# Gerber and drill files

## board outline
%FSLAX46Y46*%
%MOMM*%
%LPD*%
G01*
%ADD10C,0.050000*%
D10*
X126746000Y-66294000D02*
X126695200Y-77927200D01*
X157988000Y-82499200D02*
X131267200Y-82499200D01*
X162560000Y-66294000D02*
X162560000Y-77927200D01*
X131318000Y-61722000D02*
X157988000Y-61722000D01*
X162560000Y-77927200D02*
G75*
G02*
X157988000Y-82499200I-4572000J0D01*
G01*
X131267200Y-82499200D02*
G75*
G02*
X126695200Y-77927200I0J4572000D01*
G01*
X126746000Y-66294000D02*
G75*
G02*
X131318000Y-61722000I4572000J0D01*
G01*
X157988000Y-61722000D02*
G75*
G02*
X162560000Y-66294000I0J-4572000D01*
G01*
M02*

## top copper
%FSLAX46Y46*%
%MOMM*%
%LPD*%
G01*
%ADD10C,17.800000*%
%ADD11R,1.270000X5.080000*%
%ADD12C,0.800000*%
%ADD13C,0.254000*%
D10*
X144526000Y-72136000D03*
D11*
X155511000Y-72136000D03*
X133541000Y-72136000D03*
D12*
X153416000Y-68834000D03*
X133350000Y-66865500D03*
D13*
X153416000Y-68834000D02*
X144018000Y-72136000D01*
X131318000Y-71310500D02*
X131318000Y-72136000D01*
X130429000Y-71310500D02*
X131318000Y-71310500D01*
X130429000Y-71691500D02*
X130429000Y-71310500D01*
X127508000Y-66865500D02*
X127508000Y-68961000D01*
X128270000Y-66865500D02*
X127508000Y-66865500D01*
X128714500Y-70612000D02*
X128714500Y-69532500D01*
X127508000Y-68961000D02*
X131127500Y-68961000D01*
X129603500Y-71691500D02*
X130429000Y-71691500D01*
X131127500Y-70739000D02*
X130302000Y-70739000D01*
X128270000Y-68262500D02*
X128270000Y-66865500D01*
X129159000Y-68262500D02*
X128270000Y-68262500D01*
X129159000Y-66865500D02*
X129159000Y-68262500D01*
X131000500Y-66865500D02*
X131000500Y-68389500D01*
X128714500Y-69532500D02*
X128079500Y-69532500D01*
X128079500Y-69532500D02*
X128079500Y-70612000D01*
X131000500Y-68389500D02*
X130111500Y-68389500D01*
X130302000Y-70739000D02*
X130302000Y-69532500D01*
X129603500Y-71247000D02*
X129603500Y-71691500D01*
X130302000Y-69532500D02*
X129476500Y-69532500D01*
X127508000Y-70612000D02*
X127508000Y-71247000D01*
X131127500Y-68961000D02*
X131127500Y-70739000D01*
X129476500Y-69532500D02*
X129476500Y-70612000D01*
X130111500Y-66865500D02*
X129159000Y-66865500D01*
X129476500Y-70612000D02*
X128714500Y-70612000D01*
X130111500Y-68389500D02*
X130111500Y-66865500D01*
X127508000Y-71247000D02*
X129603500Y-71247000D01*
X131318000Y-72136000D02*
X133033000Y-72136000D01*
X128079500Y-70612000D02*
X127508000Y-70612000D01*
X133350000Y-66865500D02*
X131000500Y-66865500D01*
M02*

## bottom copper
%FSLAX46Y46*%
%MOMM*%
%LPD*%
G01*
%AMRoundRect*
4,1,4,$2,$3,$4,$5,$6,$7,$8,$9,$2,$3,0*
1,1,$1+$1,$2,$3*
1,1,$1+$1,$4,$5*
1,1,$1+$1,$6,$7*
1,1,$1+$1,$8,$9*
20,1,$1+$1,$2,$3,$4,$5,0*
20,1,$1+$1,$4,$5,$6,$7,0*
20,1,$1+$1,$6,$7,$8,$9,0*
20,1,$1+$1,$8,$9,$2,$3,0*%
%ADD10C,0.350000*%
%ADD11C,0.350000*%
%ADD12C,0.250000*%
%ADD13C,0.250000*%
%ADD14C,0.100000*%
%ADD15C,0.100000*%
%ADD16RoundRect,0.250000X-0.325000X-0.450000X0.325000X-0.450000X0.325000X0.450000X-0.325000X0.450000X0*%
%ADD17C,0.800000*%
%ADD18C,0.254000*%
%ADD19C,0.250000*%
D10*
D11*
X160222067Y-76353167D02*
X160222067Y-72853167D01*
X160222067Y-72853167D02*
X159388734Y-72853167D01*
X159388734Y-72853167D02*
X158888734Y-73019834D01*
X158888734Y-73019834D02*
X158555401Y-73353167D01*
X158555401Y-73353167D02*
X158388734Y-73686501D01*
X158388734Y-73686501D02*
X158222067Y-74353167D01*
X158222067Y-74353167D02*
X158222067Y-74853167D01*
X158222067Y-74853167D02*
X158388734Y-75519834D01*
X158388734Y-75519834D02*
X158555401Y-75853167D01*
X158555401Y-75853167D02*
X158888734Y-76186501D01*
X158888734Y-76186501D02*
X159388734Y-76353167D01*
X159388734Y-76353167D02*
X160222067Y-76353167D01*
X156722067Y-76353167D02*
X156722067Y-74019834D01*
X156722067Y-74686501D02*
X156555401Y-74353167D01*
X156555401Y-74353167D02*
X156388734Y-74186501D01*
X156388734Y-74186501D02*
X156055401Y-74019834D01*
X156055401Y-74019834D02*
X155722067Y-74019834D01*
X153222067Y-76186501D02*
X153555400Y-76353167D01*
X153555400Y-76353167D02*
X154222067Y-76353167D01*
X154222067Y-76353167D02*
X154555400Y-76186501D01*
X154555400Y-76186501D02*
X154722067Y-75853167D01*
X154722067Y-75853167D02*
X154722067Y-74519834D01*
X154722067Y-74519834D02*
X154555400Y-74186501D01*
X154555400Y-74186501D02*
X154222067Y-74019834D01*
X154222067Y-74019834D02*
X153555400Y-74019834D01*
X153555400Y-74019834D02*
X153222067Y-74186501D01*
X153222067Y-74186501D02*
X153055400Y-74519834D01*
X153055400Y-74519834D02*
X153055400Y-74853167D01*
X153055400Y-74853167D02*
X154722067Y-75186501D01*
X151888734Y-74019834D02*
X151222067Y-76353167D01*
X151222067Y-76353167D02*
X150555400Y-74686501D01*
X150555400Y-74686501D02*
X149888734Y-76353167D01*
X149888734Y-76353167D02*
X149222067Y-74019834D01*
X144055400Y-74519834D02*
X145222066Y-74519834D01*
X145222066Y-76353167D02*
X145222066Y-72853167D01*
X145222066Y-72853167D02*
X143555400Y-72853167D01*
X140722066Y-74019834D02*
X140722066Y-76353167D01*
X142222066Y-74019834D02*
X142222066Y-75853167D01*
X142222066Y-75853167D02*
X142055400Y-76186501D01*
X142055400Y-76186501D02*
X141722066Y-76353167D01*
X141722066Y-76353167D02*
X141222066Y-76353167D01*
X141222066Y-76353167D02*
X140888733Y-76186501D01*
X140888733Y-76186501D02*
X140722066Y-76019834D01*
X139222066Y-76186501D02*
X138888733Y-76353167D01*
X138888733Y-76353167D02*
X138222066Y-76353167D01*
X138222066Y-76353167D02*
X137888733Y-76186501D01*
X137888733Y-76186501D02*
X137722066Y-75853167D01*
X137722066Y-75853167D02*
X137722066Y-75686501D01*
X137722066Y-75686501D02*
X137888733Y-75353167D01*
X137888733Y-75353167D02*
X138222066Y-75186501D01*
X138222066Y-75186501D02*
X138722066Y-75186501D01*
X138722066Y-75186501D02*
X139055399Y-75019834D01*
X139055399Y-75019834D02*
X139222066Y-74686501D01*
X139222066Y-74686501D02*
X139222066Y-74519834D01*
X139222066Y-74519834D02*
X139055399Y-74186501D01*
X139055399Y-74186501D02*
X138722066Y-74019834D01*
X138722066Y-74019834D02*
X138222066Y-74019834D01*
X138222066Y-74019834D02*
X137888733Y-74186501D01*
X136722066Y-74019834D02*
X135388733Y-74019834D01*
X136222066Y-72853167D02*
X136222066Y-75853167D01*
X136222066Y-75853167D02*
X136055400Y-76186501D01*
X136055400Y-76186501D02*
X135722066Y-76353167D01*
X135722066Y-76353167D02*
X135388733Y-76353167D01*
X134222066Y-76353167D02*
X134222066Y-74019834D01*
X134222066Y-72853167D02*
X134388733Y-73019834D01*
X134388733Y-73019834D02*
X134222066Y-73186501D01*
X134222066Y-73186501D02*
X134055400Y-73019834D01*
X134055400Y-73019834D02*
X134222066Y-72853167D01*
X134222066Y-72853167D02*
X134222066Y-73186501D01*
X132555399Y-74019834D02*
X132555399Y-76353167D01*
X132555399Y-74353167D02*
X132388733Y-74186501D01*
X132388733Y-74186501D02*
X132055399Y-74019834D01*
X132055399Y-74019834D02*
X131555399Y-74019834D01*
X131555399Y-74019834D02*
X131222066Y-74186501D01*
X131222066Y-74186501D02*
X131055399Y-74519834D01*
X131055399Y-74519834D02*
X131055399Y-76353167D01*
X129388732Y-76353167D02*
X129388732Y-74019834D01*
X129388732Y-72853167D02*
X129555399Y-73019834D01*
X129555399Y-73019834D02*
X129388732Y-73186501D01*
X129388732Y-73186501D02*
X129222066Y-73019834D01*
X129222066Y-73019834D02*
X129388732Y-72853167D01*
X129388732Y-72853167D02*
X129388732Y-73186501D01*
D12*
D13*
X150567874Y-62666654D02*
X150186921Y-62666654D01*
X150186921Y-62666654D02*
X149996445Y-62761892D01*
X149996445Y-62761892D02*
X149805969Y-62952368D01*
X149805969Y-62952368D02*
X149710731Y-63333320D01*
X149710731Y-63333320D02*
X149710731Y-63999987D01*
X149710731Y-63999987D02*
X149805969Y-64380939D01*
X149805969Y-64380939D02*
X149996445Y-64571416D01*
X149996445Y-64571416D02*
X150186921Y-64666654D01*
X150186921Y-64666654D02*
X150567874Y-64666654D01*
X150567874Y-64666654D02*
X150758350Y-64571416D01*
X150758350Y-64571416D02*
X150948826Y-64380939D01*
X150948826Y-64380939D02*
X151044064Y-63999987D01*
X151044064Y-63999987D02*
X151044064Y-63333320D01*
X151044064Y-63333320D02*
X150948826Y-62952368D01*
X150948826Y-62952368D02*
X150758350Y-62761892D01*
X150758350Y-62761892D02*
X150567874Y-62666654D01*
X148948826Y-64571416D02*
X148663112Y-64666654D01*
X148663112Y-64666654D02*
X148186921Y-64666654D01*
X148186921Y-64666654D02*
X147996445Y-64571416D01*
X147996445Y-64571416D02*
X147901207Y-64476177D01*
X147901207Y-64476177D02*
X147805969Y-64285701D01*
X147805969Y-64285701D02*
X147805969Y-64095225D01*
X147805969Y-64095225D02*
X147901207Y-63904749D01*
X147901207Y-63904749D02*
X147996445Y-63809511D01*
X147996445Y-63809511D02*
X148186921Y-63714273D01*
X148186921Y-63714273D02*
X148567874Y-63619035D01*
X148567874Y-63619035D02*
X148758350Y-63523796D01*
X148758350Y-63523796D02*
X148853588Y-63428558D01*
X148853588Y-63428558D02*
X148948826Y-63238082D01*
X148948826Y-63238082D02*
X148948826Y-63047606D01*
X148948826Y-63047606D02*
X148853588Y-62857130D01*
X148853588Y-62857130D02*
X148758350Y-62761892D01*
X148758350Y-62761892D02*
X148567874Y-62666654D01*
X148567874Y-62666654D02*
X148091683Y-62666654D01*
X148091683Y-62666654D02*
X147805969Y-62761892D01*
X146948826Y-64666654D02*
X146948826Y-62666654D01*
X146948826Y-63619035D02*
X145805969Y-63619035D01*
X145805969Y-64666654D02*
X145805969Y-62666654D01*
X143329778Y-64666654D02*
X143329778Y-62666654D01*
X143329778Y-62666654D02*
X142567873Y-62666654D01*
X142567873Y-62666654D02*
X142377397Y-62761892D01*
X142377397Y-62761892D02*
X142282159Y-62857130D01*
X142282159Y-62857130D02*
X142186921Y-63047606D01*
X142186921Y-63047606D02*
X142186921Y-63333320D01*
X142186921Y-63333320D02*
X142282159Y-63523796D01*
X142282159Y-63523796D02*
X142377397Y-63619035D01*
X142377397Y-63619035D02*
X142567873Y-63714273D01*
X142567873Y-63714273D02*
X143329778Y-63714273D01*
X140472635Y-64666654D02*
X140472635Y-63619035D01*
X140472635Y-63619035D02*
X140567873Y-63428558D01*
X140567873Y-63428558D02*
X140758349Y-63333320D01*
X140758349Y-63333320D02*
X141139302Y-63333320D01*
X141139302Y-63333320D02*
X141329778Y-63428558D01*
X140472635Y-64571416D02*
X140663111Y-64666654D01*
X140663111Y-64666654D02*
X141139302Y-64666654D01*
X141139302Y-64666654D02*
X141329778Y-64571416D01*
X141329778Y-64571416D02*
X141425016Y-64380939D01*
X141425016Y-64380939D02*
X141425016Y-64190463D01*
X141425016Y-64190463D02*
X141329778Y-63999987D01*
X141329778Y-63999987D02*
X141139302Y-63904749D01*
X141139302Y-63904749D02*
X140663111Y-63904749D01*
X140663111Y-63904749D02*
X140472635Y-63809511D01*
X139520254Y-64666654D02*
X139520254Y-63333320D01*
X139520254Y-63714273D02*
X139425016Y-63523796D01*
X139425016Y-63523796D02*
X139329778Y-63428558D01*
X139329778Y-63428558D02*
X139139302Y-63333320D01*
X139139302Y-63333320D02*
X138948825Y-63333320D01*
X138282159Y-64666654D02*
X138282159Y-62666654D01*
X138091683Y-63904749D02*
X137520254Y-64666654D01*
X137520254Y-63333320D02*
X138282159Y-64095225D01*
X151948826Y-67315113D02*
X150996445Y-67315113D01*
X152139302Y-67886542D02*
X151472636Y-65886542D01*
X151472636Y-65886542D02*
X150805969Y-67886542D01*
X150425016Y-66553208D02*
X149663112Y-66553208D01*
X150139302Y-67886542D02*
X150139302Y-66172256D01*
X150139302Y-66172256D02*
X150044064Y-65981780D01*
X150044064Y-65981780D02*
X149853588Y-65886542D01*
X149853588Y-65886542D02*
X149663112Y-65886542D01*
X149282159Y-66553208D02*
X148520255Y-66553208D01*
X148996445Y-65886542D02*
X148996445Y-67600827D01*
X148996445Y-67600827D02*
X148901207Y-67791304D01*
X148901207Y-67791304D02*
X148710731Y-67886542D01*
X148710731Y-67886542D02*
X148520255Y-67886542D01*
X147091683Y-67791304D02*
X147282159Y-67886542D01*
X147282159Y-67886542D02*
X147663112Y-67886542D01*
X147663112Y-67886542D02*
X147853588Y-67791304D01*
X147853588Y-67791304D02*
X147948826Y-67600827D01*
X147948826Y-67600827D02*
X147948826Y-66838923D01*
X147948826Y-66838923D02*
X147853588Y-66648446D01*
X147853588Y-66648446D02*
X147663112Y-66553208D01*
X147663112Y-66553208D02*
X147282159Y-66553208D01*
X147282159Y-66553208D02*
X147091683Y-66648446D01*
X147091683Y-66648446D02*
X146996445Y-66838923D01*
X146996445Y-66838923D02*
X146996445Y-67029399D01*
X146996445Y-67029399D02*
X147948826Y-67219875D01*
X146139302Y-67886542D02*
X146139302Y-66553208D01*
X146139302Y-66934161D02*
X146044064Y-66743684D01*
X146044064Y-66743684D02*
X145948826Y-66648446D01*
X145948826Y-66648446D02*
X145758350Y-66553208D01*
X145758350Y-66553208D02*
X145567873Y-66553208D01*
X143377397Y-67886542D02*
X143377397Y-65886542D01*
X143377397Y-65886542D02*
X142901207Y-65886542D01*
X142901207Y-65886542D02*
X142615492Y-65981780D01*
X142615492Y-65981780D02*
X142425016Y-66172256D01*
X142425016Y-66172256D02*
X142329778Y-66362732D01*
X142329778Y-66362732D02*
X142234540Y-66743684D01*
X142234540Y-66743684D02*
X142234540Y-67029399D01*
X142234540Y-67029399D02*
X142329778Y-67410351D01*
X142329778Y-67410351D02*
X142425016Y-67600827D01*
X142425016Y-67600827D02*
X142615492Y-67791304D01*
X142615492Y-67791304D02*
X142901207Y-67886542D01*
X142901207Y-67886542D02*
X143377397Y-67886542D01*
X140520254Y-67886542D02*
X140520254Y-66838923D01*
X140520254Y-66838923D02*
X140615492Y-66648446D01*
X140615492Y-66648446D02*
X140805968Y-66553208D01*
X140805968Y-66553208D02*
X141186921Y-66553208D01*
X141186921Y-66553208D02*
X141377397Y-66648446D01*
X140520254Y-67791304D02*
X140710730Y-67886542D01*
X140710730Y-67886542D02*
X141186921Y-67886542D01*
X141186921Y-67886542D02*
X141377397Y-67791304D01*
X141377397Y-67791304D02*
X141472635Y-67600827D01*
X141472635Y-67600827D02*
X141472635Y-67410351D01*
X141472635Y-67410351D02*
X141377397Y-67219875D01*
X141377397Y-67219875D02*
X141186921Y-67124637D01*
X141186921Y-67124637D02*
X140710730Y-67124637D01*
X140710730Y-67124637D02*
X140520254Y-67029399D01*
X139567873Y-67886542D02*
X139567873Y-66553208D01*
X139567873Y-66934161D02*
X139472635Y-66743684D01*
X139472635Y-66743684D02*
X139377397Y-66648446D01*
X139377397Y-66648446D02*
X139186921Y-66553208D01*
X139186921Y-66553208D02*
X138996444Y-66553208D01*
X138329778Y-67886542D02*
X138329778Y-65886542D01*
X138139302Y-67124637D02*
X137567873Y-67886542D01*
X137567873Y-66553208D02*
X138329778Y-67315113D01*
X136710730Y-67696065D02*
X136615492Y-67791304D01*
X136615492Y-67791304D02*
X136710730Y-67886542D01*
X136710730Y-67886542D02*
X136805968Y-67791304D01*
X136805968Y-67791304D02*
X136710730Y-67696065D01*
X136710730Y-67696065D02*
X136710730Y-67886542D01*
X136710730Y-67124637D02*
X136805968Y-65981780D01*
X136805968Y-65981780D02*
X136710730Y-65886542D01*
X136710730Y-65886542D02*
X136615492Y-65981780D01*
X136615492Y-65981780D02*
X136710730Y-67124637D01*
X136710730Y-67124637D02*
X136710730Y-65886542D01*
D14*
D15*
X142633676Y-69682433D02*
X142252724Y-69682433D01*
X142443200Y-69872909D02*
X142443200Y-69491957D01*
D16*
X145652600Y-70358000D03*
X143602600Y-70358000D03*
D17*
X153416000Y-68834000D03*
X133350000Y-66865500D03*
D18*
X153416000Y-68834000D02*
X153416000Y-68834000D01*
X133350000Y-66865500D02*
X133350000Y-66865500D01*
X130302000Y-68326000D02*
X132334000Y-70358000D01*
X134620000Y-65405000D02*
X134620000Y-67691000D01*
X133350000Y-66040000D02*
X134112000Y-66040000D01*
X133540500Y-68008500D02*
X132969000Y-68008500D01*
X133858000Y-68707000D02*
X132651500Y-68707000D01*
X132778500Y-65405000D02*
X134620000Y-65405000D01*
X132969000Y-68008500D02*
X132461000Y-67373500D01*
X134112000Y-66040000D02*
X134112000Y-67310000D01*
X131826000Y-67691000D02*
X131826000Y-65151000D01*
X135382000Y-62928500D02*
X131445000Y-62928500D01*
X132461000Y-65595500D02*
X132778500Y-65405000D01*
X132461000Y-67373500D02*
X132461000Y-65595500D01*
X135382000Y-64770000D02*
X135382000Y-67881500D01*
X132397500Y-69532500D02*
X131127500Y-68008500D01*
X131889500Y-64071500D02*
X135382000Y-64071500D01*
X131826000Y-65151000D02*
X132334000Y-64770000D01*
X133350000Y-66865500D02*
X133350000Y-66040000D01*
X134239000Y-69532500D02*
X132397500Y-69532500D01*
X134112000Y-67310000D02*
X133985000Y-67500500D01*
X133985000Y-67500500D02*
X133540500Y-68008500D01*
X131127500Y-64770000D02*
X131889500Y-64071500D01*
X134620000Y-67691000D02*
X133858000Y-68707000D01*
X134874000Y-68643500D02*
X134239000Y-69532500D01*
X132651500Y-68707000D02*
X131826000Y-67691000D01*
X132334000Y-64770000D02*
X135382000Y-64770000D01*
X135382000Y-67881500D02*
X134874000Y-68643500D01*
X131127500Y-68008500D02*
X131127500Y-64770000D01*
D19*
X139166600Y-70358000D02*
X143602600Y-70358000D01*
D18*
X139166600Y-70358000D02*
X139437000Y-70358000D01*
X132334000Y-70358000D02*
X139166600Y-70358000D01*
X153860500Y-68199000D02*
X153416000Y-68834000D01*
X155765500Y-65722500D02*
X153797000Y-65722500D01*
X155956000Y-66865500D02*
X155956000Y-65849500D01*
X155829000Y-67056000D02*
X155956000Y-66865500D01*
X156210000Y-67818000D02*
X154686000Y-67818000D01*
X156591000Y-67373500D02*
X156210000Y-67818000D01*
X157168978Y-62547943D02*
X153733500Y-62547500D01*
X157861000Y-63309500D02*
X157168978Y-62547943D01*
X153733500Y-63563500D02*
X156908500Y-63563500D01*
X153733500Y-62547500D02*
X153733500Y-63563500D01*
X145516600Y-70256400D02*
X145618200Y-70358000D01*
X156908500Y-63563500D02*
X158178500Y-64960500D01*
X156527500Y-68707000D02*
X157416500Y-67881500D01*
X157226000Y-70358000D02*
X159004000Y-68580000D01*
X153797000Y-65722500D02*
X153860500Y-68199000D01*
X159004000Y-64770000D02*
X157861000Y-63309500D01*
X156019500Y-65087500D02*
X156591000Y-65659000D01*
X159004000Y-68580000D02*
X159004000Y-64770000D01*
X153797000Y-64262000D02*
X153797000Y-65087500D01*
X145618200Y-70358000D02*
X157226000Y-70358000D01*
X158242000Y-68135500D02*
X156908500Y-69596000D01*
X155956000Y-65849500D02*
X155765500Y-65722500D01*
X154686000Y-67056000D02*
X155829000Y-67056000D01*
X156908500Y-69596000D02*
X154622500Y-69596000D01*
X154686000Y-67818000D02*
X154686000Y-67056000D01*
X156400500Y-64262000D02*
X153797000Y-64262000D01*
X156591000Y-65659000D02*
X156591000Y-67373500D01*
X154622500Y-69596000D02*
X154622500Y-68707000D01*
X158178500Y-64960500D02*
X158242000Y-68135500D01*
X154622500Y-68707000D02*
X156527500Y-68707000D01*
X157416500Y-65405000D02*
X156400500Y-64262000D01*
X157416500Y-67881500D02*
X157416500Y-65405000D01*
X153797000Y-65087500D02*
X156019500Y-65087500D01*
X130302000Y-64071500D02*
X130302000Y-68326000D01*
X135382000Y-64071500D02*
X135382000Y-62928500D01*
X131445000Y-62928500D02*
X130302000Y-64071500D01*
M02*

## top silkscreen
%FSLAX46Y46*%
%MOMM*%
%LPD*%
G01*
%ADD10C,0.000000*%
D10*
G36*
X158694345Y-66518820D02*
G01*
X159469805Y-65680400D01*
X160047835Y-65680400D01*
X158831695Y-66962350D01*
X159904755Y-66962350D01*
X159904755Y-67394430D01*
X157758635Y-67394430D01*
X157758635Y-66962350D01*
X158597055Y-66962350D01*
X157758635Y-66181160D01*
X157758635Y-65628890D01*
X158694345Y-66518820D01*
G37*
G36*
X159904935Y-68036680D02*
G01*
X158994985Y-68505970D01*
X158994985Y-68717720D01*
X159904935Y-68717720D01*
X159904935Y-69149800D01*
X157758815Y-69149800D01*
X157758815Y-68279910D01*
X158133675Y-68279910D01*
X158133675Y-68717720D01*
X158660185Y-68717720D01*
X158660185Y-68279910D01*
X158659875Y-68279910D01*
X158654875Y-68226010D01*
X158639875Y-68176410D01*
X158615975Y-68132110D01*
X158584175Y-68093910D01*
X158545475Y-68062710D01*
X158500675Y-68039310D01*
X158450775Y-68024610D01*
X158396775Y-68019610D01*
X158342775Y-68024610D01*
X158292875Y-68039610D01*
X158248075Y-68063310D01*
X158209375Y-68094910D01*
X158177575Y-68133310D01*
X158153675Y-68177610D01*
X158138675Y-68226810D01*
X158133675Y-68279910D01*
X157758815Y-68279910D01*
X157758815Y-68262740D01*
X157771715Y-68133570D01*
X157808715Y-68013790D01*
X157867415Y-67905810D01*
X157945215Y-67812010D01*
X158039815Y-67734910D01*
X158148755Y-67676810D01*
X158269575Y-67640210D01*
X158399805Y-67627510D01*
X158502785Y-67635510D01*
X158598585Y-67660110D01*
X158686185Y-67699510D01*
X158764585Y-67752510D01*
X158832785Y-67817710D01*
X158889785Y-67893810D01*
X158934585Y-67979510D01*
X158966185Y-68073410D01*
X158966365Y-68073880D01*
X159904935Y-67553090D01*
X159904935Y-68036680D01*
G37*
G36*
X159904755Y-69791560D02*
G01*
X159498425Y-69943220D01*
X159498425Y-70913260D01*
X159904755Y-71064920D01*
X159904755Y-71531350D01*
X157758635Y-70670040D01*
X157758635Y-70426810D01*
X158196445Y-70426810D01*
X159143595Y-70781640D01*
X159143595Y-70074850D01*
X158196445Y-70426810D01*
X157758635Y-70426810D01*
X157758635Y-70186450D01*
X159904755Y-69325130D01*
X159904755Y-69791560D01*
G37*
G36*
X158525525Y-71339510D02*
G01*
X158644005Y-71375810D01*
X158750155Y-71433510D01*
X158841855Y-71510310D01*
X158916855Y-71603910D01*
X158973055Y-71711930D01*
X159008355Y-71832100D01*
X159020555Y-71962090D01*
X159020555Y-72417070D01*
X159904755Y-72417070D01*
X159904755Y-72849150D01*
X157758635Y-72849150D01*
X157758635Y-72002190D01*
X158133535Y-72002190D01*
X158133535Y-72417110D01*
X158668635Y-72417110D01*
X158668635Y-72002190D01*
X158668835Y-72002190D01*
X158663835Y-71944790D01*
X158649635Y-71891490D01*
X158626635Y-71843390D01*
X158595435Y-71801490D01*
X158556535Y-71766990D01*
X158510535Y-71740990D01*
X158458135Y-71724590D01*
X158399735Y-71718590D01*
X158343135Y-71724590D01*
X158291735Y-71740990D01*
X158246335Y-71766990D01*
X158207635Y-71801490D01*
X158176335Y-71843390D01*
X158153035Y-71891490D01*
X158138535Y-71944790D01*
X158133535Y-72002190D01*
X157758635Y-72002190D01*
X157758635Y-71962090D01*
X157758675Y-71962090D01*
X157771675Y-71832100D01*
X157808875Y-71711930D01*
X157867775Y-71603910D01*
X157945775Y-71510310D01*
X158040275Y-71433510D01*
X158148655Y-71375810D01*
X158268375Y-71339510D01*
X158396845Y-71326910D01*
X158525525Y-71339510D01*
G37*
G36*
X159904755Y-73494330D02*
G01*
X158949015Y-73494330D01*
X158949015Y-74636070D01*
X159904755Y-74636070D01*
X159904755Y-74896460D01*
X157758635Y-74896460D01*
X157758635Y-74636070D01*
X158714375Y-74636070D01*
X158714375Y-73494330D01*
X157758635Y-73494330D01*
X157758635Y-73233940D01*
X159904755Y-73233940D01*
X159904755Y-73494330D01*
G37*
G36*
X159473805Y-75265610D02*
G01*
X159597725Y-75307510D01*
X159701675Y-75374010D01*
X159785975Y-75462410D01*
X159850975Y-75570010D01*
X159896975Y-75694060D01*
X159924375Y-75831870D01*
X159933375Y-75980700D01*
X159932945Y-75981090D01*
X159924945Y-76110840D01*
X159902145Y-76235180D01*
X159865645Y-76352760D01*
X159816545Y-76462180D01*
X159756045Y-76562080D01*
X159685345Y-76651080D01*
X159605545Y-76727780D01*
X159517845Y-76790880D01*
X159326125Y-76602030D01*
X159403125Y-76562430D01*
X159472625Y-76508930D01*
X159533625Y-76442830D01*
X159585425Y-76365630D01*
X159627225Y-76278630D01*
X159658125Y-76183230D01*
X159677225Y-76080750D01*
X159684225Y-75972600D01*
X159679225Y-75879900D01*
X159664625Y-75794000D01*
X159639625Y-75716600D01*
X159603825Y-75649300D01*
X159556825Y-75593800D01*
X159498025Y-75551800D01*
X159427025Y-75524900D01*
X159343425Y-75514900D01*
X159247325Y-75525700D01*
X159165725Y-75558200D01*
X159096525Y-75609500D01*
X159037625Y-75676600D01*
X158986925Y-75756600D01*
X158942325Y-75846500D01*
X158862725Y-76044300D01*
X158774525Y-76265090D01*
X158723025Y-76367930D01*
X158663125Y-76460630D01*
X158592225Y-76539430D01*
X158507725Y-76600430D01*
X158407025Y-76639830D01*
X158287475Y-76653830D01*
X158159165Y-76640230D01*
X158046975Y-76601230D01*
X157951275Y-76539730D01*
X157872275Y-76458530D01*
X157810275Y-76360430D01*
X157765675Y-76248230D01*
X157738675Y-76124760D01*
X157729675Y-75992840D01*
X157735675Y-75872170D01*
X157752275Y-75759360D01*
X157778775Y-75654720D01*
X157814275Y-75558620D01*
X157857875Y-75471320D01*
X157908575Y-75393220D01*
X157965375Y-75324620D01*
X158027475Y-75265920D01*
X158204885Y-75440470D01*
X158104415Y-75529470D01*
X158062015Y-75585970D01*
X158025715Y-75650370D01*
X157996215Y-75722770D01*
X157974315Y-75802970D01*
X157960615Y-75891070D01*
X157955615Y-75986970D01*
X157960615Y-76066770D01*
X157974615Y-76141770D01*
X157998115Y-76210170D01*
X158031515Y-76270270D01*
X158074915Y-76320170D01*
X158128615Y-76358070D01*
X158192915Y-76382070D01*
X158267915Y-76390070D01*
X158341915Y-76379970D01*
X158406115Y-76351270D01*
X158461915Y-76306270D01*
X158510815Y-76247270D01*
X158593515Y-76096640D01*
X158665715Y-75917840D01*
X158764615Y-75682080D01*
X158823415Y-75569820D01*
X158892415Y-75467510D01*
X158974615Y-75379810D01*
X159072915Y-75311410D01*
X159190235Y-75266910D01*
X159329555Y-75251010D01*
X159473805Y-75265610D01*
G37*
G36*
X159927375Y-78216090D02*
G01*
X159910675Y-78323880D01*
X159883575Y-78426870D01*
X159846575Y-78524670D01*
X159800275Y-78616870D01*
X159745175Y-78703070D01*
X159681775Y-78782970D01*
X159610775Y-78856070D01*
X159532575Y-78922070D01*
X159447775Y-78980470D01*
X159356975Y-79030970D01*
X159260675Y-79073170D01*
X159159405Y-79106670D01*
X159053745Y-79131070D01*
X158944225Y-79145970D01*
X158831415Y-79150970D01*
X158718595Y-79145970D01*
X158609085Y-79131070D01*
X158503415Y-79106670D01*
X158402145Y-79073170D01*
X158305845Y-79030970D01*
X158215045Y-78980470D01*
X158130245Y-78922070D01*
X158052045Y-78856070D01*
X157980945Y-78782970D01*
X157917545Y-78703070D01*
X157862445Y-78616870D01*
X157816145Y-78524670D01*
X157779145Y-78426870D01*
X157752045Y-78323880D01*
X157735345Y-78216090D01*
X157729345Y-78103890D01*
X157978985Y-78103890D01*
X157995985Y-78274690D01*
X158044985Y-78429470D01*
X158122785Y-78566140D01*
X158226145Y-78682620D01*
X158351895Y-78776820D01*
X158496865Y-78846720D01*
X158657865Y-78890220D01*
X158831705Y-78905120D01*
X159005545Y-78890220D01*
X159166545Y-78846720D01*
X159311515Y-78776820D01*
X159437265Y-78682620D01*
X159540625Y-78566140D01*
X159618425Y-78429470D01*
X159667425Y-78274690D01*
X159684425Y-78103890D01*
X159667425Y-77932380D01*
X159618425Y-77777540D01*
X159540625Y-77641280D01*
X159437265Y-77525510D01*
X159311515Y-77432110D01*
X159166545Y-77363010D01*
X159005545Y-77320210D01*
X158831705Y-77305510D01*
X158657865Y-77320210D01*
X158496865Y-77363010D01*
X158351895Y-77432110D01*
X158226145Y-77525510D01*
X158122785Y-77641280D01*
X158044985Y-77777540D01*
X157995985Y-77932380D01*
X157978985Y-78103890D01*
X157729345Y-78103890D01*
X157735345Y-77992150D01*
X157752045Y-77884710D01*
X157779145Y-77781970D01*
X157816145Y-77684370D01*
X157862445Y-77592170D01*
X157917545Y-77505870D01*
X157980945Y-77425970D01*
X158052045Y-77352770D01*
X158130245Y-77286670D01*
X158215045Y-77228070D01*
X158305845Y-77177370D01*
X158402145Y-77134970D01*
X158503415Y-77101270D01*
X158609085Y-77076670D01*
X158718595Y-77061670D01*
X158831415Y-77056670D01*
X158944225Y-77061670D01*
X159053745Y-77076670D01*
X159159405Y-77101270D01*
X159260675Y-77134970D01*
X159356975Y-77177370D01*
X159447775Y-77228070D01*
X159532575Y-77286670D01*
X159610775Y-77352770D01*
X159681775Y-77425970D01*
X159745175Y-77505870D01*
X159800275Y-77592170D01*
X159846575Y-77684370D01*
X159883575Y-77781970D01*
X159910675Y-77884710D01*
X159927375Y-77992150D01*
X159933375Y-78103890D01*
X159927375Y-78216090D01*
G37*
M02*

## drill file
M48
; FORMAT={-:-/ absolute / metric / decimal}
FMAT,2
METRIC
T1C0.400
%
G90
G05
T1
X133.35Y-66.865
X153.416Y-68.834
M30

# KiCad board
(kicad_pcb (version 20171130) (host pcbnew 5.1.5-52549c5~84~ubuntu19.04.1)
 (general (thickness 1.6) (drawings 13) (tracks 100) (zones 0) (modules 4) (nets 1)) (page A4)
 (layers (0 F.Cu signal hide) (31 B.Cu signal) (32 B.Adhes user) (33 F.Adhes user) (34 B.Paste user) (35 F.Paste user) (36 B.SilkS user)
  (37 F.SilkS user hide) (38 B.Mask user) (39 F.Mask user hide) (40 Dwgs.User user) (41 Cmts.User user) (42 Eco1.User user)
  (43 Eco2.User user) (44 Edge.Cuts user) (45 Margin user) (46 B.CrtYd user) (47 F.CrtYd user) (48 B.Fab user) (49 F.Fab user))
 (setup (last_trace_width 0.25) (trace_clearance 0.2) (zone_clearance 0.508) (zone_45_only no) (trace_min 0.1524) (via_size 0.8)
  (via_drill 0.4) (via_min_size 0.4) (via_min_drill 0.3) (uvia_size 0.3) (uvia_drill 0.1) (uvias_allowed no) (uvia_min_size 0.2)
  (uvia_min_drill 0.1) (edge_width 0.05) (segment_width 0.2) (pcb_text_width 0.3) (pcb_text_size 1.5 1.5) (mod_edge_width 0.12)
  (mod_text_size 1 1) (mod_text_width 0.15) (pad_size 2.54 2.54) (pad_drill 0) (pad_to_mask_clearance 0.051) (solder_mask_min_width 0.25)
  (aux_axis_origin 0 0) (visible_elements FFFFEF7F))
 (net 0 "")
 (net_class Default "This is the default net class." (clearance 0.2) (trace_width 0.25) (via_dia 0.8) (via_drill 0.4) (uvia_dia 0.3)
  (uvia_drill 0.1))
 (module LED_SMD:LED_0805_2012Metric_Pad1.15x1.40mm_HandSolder (layer B.Cu) (at 144.6276 70.358)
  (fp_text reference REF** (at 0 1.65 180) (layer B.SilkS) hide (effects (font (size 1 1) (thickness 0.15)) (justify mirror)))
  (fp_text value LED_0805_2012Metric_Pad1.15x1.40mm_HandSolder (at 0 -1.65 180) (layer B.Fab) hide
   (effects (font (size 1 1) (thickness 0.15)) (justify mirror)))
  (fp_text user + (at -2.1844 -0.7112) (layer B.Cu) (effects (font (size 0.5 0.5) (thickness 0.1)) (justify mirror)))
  (pad 2 smd roundrect (at 1.025 0) (size 1.15 1.4) (layers B.Cu B.Paste B.Mask) (roundrect_rratio 0.217391))
  (pad 1 smd roundrect (at -1.025 0) (size 1.15 1.4) (layers B.Cu B.Paste B.Mask) (roundrect_rratio 0.217391)))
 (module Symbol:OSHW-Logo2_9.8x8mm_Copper (layer F.Cu) (at 131.572 79.502)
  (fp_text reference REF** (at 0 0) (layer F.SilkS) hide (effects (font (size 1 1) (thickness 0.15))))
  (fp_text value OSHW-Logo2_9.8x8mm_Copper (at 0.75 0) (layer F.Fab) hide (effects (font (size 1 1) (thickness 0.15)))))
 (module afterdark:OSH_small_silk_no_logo (layer F.Cu) (at 151.638 72.39 90)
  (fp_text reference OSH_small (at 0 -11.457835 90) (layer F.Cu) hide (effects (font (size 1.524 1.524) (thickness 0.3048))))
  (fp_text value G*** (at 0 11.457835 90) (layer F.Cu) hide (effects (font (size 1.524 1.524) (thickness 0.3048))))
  (fp_poly
   (pts (xy 6.76111 6.120635) (xy 6.20884 6.120635) (xy 5.42765 6.959055) (xy 5.42765 6.120635) (xy 4.99557 6.120635) (xy 4.99557 8.266755)
    (xy 5.42765 8.266755) (xy 5.42765 7.193695) (xy 6.7096 8.409835) (xy 6.7096 7.831805) (xy 5.87118 7.056345) (xy 6.76111 6.120635))
   (layer F.SilkS) (width 0))
  (fp_poly
   (pts (xy 4.31659 7.328185) (xy 4.11009 7.022185) (xy 3.67228 7.022185) (xy 3.67228 6.495675) (xy 4.11009 6.495675) (xy 4.16319 6.500675)
    (xy 4.21239 6.515675) (xy 4.25669 6.539575) (xy 4.29509 6.571375) (xy 4.32669 6.610075) (xy 4.35039 6.654875) (xy 4.36539 6.704775)
    (xy 4.37039 6.758775) (xy 4.36539 6.812775) (xy 4.35069 6.862675) (xy 4.32729 6.907475) (xy 4.29609 6.946175) (xy 4.25789 6.977975)
    (xy 4.21359 7.001875) (xy 4.16399 7.016875) (xy 4.11009 7.021875) (xy 4.11009 7.022185) (xy 4.31659 7.328185) (xy 4.41049 7.296585)
    (xy 4.49619 7.251785) (xy 4.57229 7.194785) (xy 4.63749 7.126585) (xy 4.69049 7.048185) (xy 4.72989 6.960585) (xy 4.75449 6.864785)
    (xy 4.76249 6.761805) (xy 4.74979 6.631575) (xy 4.71319 6.510755) (xy 4.65509 6.401815) (xy 4.57799 6.307215) (xy 4.48419 6.229415)
    (xy 4.37621 6.170715) (xy 4.25643 6.133715) (xy 4.12726 6.120815) (xy 3.2402 6.120815) (xy 3.2402 8.266935) (xy 3.67228 8.266935)
    (xy 3.67228 7.356985) (xy 3.88403 7.356985) (xy 4.35332 8.266935) (xy 4.83691 8.266935) (xy 4.31612 7.328365) (xy 4.31659 7.328185))
   (layer F.SilkS) (width 0))
  (fp_poly
   (pts (xy 2.59844 8.266755) (xy 1.96319 6.558445) (xy 2.31515 7.505595) (xy 1.60836 7.505595) (xy 1.96319 6.558445) (xy 2.59844 8.266755)
    (xy 3.06487 8.266755) (xy 2.20355 6.120635) (xy 1.71996 6.120635) (xy 0.85865 8.266755) (xy 1.32508 8.266755) (xy 1.47674 7.860425)
    (xy 2.44678 7.860425) (xy 2.59844 8.266755))
   (layer F.SilkS) (width 0))
  (fp_poly
   (pts (xy 0.42791 6.120635) (xy -0.02711 6.495535) (xy 0.38781 6.495535) (xy 0.44521 6.500535) (xy 0.49851 6.515035) (xy 0.54661 6.538335)
    (xy 0.58851 6.569635) (xy 0.62301 6.608335) (xy 0.64901 6.653735) (xy 0.66541 6.705135) (xy 0.67141 6.761735) (xy 0.66541 6.820135)
    (xy 0.64901 6.872535) (xy 0.62301 6.918535) (xy 0.58851 6.957435) (xy 0.54661 6.988635) (xy 0.49851 7.011635) (xy 0.44521 7.025835)
    (xy 0.38781 7.030835) (xy 0.38781 7.030635) (xy -0.02711 7.030635) (xy -0.02711 6.495535) (xy 0.42791 6.120635) (xy -0.45915 6.120635)
    (xy -0.45915 8.266755) (xy -0.02707 8.266755) (xy -0.02707 7.382555) (xy 0.42791 7.382555) (xy 0.5579 7.370355) (xy 0.67807 7.335055)
    (xy 0.78609 7.278855) (xy 0.87969 7.203855) (xy 0.95649 7.112155) (xy 1.01419 7.006005) (xy 1.05049 6.887525) (xy 1.06309 6.758845)
    (xy 1.05049 6.630375) (xy 1.01419 6.510655) (xy 0.95649 6.402275) (xy 0.87969 6.307775) (xy 0.78609 6.229775) (xy 0.67807 6.170875)
    (xy 0.5579 6.133675) (xy 0.42791 6.120675) (xy 0.42791 6.120635))
   (layer F.SilkS) (width 0))
  (fp_poly
   (pts (xy -1.10433 6.120635) (xy -1.10433 7.076375) (xy -2.24607 7.076375) (xy -2.24607 6.120635) (xy -2.50646 6.120635)
    (xy -2.50646 8.266755) (xy -2.24607 8.266755) (xy -2.24607 7.311015) (xy -1.10433 7.311015) (xy -1.10433 8.266755)
    (xy -0.84394 8.266755) (xy -0.84394 6.120635) (xy -1.10433 6.120635))
   (layer F.SilkS) (width 0))
  (fp_poly
   (pts (xy -3.5907 8.295375) (xy -3.44187 8.286375) (xy -3.30406 8.258975) (xy -3.18001 8.212975) (xy -3.07241 8.147975)
    (xy -2.98401 8.063675) (xy -2.91751 7.959725) (xy -2.87561 7.835805) (xy -2.86101 7.691555) (xy -2.87691 7.552235)
    (xy -2.92141 7.434915) (xy -2.98981 7.336615) (xy -3.07751 7.254415) (xy -3.17982 7.185415) (xy -3.29208 7.126615)
    (xy -3.52784 7.027715) (xy -3.70664 6.955515) (xy -3.85727 6.872815) (xy -3.91627 6.823915) (xy -3.96127 6.768115)
    (xy -3.98997 6.703915) (xy -4.00007 6.629915) (xy -3.99207 6.554915) (xy -3.96807 6.490615) (xy -3.93017 6.436915)
    (xy -3.88027 6.393515) (xy -3.82017 6.360115) (xy -3.75177 6.336615) (xy -3.67677 6.322615) (xy -3.59697 6.317615)
    (xy -3.50107 6.322615) (xy -3.41297 6.336315) (xy -3.33277 6.358215) (xy -3.26037 6.387715) (xy -3.19597 6.424015)
    (xy -3.13947 6.466415) (xy -3.05047 6.566885) (xy -2.87592 6.389475) (xy -2.93462 6.327375) (xy -3.00322 6.270575)
    (xy -3.08132 6.219875) (xy -3.16862 6.176275) (xy -3.26472 6.140775) (xy -3.36936 6.114275) (xy -3.48217 6.097675)
    (xy -3.60284 6.091675) (xy -3.73476 6.100675) (xy -3.85823 6.127675) (xy -3.97043 6.172275) (xy -4.06853 6.234275)
    (xy -4.14973 6.313275) (xy -4.21123 6.408975) (xy -4.25023 6.521165) (xy -4.26383 6.649475) (xy -4.24983 6.769025)
    (xy -4.21043 6.869725) (xy -4.14943 6.954225) (xy -4.07063 7.025125) (xy -3.97793 7.085025) (xy -3.87509 7.136525) (xy -3.6543 7.224725)
    (xy -3.4565 7.304325) (xy -3.3666 7.348925) (xy -3.2866 7.399625) (xy -3.2195 7.458525) (xy -3.1682 7.527725) (xy -3.1357 7.609325)
    (xy -3.1249 7.705425) (xy -3.1349 7.789025) (xy -3.1618 7.860025) (xy -3.2038 7.918825) (xy -3.2593 7.965825) (xy -3.3266 8.001625)
    (xy -3.404 8.026625) (xy -3.4899 8.041225) (xy -3.5826 8.046225) (xy -3.69075 8.039225) (xy -3.79323 8.020125) (xy -3.88863 7.989225)
    (xy -3.97563 7.947425) (xy -4.05283 7.895625) (xy -4.11893 7.834625) (xy -4.17243 7.765125) (xy -4.21203 7.688125)
    (xy -4.40088 7.879845) (xy -4.33778 7.967545) (xy -4.26108 8.047345) (xy -4.17208 8.118045) (xy -4.07218 8.178545)
    (xy -3.96276 8.227645) (xy -3.84518 8.264145) (xy -3.72084 8.286945) (xy -3.59109 8.294945) (xy -3.5907 8.295375))
   (layer F.SilkS) (width 0))
  (fp_poly
   (pts (xy -5.71389 8.295375) (xy -5.71389 8.046425) (xy -5.88469 8.029425) (xy -6.03947 7.980425) (xy -6.17614 7.902625)
    (xy -6.29262 7.799265) (xy -6.38682 7.673515) (xy -6.45672 7.528545) (xy -6.50022 7.367545) (xy -6.51512 7.193705)
    (xy -6.50022 7.019865) (xy -6.45672 6.858865) (xy -6.38682 6.713895) (xy -6.29262 6.588145) (xy -6.17614 6.484785)
    (xy -6.03947 6.406985) (xy -5.88469 6.357985) (xy -5.71389 6.340985) (xy -5.54238 6.357985) (xy -5.38754 6.406985)
    (xy -5.25128 6.484785) (xy -5.13551 6.588145) (xy -5.04211 6.713895) (xy -4.97301 6.858865) (xy -4.93021 7.019865)
    (xy -4.91551 7.193705) (xy -4.93021 7.367545) (xy -4.97301 7.528545) (xy -5.04211 7.673515) (xy -5.13551 7.799265)
    (xy -5.25128 7.902625) (xy -5.38754 7.980425) (xy -5.54238 8.029425) (xy -5.71389 8.046425) (xy -5.71389 8.295375)
    (xy -5.60215 8.289375) (xy -5.49471 8.272675) (xy -5.39197 8.245575) (xy -5.29437 8.208575) (xy -5.20217 8.162275)
    (xy -5.11587 8.107175) (xy -5.03597 8.043775) (xy -4.96277 7.972775) (xy -4.89667 7.894575) (xy -4.83807 7.809775)
    (xy -4.78737 7.718975) (xy -4.74497 7.622675) (xy -4.71127 7.521405) (xy -4.68667 7.415745) (xy -4.67167 7.306225)
    (xy -4.66667 7.193415) (xy -4.67167 7.080595) (xy -4.68667 6.971085) (xy -4.71127 6.865415) (xy -4.74497 6.764145)
    (xy -4.78737 6.667845) (xy -4.83807 6.577045) (xy -4.89667 6.492245) (xy -4.96277 6.414045) (xy -5.03597 6.342945)
    (xy -5.11587 6.279545) (xy -5.20217 6.224445) (xy -5.29437 6.178145) (xy -5.39197 6.141145) (xy -5.49471 6.114045)
    (xy -5.60215 6.097345) (xy -5.71389 6.091345) (xy -5.82609 6.097345) (xy -5.93388 6.114045) (xy -6.03687 6.141145)
    (xy -6.13467 6.178145) (xy -6.22687 6.224445) (xy -6.31307 6.279545) (xy -6.39297 6.342945) (xy -6.46607 6.414045)
    (xy -6.53207 6.492245) (xy -6.59047 6.577045) (xy -6.64097 6.667845) (xy -6.68317 6.764145) (xy -6.71667 6.865415)
    (xy -6.74107 6.971085) (xy -6.75597 7.080595) (xy -6.76097 7.193415) (xy -6.75597 7.306225) (xy -6.74107 7.415745)
    (xy -6.71667 7.521405) (xy -6.68317 7.622675) (xy -6.64097 7.718975) (xy -6.59047 7.809775) (xy -6.53207 7.894575)
    (xy -6.46607 7.972775) (xy -6.39297 8.043775) (xy -6.31307 8.107175) (xy -6.22687 8.162275) (xy -6.13467 8.208575)
    (xy -6.03687 8.245575) (xy -5.93388 8.272675) (xy -5.82609 8.289375) (xy -5.71389 8.295375))
   (layer F.SilkS) (width 0)))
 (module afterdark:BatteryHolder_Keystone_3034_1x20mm (layer F.Cu) (at 144.526 72.136)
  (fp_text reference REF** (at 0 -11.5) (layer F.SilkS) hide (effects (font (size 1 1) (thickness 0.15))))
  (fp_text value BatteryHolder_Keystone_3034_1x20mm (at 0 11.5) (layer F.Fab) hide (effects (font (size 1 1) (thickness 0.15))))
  (pad 2 smd circle (at 0 0) (size 17.8 17.8) (layers F.Cu F.Mask))
  (pad 1 smd rect (at 10.985 0) (size 1.27 5.08) (layers F.Cu F.Paste F.Mask))
  (pad 1 smd rect (at -10.985 0) (size 1.27 5.08) (layers F.Cu F.Paste F.Mask)))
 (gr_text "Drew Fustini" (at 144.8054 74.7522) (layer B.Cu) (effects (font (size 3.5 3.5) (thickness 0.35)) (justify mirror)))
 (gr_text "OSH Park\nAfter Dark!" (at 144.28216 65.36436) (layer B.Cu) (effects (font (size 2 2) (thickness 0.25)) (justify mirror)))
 (gr_line (start 126.746 66.294) (end 126.6952 77.9272) (layer Edge.Cuts) (width 0.05))
 (gr_line (start 157.988 82.4992) (end 131.2672 82.4992) (layer Edge.Cuts) (width 0.05))
 (gr_line (start 162.56 66.294) (end 162.56 77.9272) (layer Edge.Cuts) (width 0.05))
 (gr_line (start 131.318 61.722) (end 157.988 61.722) (layer Edge.Cuts) (width 0.05))
 (gr_arc (start 157.988 77.9272) (end 157.988 82.4992) (angle -90) (layer Edge.Cuts) (width 0.05))
 (gr_arc (start 131.2672 77.9272) (end 126.6952 77.9272) (angle -90) (layer Edge.Cuts) (width 0.05))
 (gr_arc (start 131.318 66.294) (end 131.318 61.722) (angle -90) (layer Edge.Cuts) (width 0.05))
 (gr_arc (start 157.988 66.294) (end 162.56 66.294) (angle -90) (layer Edge.Cuts) (width 0.05))
 (segment (start 153.416 68.834) (end 153.416 68.834) (width 0.254) (layer B.Cu) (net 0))
 (via (at 153.416 68.834) (size 0.8) (drill 0.4) (layers F.Cu B.Cu) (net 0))
 (segment (start 153.416 68.834) (end 144.018 72.136) (width 0.254) (layer F.Cu) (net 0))
 (segment (start 131.318 71.3105) (end 131.318 72.136) (width 0.254) (layer F.Cu) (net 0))
 (segment (start 130.429 71.3105) (end 131.318 71.3105) (width 0.254) (layer F.Cu) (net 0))
 (segment (start 130.429 71.6915) (end 130.429 71.3105) (width 0.254) (layer F.Cu) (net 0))
 (segment (start 127.508 66.8655) (end 127.508 68.961) (width 0.254) (layer F.Cu) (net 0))
 (segment (start 128.27 66.8655) (end 127.508 66.8655) (width 0.254) (layer F.Cu) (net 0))
 (segment (start 128.7145 70.612) (end 128.7145 69.5325) (width 0.254) (layer F.Cu) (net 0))
 (segment (start 127.508 68.961) (end 131.1275 68.961) (width 0.254) (layer F.Cu) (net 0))
 (segment (start 129.6035 71.6915) (end 130.429 71.6915) (width 0.254) (layer F.Cu) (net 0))
 (segment (start 131.1275 70.739) (end 130.302 70.739) (width 0.254) (layer F.Cu) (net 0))
 (segment (start 128.27 68.2625) (end 128.27 66.8655) (width 0.254) (layer F.Cu) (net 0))
 (segment (start 129.159 68.2625) (end 128.27 68.2625) (width 0.254) (layer F.Cu) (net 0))
 (segment (start 129.159 66.8655) (end 129.159 68.2625) (width 0.254) (layer F.Cu) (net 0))
 (segment (start 131.0005 66.8655) (end 131.0005 68.3895) (width 0.254) (layer F.Cu) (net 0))
 (segment (start 128.7145 69.5325) (end 128.0795 69.5325) (width 0.254) (layer F.Cu) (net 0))
 (segment (start 128.0795 69.5325) (end 128.0795 70.612) (width 0.254) (layer F.Cu) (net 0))
 (segment (start 131.0005 68.3895) (end 130.1115 68.3895) (width 0.254) (layer F.Cu) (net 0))
 (segment (start 130.302 70.739) (end 130.302 69.5325) (width 0.254) (layer F.Cu) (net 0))
 (segment (start 129.6035 71.247) (end 129.6035 71.6915) (width 0.254) (layer F.Cu) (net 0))
 (segment (start 130.302 69.5325) (end 129.4765 69.5325) (width 0.254) (layer F.Cu) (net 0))
 (segment (start 127.508 70.612) (end 127.508 71.247) (width 0.254) (layer F.Cu) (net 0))
 (segment (start 131.1275 68.961) (end 131.1275 70.739) (width 0.254) (layer F.Cu) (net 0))
 (segment (start 129.4765 69.5325) (end 129.4765 70.612) (width 0.254) (layer F.Cu) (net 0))
 (segment (start 130.1115 66.8655) (end 129.159 66.8655) (width 0.254) (layer F.Cu) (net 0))
 (segment (start 129.4765 70.612) (end 128.7145 70.612) (width 0.254) (layer F.Cu) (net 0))
 (segment (start 130.1115 68.3895) (end 130.1115 66.8655) (width 0.254) (layer F.Cu) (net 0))
 (segment (start 127.508 71.247) (end 129.6035 71.247) (width 0.254) (layer F.Cu) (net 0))
 (segment (start 131.318 72.136) (end 133.033 72.136) (width 0.254) (layer F.Cu) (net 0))
 (segment (start 128.0795 70.612) (end 127.508 70.612) (width 0.254) (layer F.Cu) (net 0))
 (segment (start 133.35 66.8655) (end 131.0005 66.8655) (width 0.254) (layer F.Cu) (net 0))
 (segment (start 133.35 66.8655) (end 133.35 66.8655) (width 0.254) (layer B.Cu) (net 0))
 (via (at 133.35 66.8655) (size 0.8) (drill 0.4) (layers F.Cu B.Cu) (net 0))
 (segment (start 130.302 68.326) (end 132.334 70.358) (width 0.254) (layer B.Cu) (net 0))
 (segment (start 134.62 65.405) (end 134.62 67.691) (width 0.254) (layer B.Cu) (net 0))
 (segment (start 133.35 66.04) (end 134.112 66.04) (width 0.254) (layer B.Cu) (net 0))
 (segment (start 133.5405 68.0085) (end 132.969 68.0085) (width 0.254) (layer B.Cu) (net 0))
 (segment (start 133.858 68.707) (end 132.6515 68.707) (width 0.254) (layer B.Cu) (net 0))
 (segment (start 132.7785 65.405) (end 134.62 65.405) (width 0.254) (layer B.Cu) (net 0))
 (segment (start 132.969 68.0085) (end 132.461 67.3735) (width 0.254) (layer B.Cu) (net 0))
 (segment (start 134.112 66.04) (end 134.112 67.31) (width 0.254) (layer B.Cu) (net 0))
 (segment (start 131.826 67.691) (end 131.826 65.151) (width 0.254) (layer B.Cu) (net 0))
 (segment (start 135.382 62.9285) (end 131.445 62.9285) (width 0.254) (layer B.Cu) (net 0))
 (segment (start 132.461 65.5955) (end 132.7785 65.405) (width 0.254) (layer B.Cu) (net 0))
 (segment (start 132.461 67.3735) (end 132.461 65.5955) (width 0.254) (layer B.Cu) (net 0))
 (segment (start 135.382 64.77) (end 135.382 67.8815) (width 0.254) (layer B.Cu) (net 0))
 (segment (start 132.3975 69.5325) (end 131.1275 68.0085) (width 0.254) (layer B.Cu) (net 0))
 (segment (start 131.8895 64.0715) (end 135.382 64.0715) (width 0.254) (layer B.Cu) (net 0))
 (segment (start 131.826 65.151) (end 132.334 64.77) (width 0.254) (layer B.Cu) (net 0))
 (segment (start 133.35 66.8655) (end 133.35 66.04) (width 0.254) (layer B.Cu) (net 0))
 (segment (start 134.239 69.5325) (end 132.3975 69.5325) (width 0.254) (layer B.Cu) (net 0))
 (segment (start 134.112 67.31) (end 133.985 67.5005) (width 0.254) (layer B.Cu) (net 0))
 (segment (start 133.985 67.5005) (end 133.5405 68.0085) (width 0.254) (layer B.Cu) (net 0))
 (segment (start 131.1275 64.77) (end 131.8895 64.0715) (width 0.254) (layer B.Cu) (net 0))
 (segment (start 134.62 67.691) (end 133.858 68.707) (width 0.254) (layer B.Cu) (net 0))
 (segment (start 134.874 68.6435) (end 134.239 69.5325) (width 0.254) (layer B.Cu) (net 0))
 (segment (start 132.6515 68.707) (end 131.826 67.691) (width 0.254) (layer B.Cu) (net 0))
 (segment (start 132.334 64.77) (end 135.382 64.77) (width 0.254) (layer B.Cu) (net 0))
 (segment (start 135.382 67.8815) (end 134.874 68.6435) (width 0.254) (layer B.Cu) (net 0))
 (segment (start 131.1275 68.0085) (end 131.1275 64.77) (width 0.254) (layer B.Cu) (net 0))
 (segment (start 139.1666 70.358) (end 143.6026 70.358) (width 0.25) (layer B.Cu) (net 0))
 (segment (start 139.1666 70.358) (end 139.437 70.358) (width 0.254) (layer B.Cu) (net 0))
 (segment (start 132.334 70.358) (end 139.1666 70.358) (width 0.254) (layer B.Cu) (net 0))
 (segment (start 153.8605 68.199) (end 153.416 68.834) (width 0.254) (layer B.Cu) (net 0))
 (segment (start 155.7655 65.7225) (end 153.797 65.7225) (width 0.254) (layer B.Cu) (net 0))
 (segment (start 155.956 66.8655) (end 155.956 65.8495) (width 0.254) (layer B.Cu) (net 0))
 (segment (start 155.829 67.056) (end 155.956 66.8655) (width 0.254) (layer B.Cu) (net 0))
 (segment (start 156.21 67.818) (end 154.686 67.818) (width 0.254) (layer B.Cu) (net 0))
 (segment (start 156.591 67.3735) (end 156.21 67.818) (width 0.254) (layer B.Cu) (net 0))
 (segment (start 157.168978 62.547943) (end 153.7335 62.5475) (width 0.254) (layer B.Cu) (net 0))
 (segment (start 157.861 63.3095) (end 157.168978 62.547943) (width 0.254) (layer B.Cu) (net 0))
 (segment (start 153.7335 63.5635) (end 156.9085 63.5635) (width 0.254) (layer B.Cu) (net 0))
 (segment (start 153.7335 62.5475) (end 153.7335 63.5635) (width 0.254) (layer B.Cu) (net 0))
 (segment (start 145.5166 70.2564) (end 145.6182 70.358) (width 0.254) (layer B.Cu) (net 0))
 (segment (start 156.9085 63.5635) (end 158.1785 64.9605) (width 0.254) (layer B.Cu) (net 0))
 (segment (start 156.5275 68.707) (end 157.4165 67.8815) (width 0.254) (layer B.Cu) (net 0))
 (segment (start 157.226 70.358) (end 159.004 68.58) (width 0.254) (layer B.Cu) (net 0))
 (segment (start 153.797 65.7225) (end 153.8605 68.199) (width 0.254) (layer B.Cu) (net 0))
 (segment (start 159.004 64.77) (end 157.861 63.3095) (width 0.254) (layer B.Cu) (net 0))
 (segment (start 156.0195 65.0875) (end 156.591 65.659) (width 0.254) (layer B.Cu) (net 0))
 (segment (start 159.004 68.58) (end 159.004 64.77) (width 0.254) (layer B.Cu) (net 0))
 (segment (start 153.797 64.262) (end 153.797 65.0875) (width 0.254) (layer B.Cu) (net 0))
 (segment (start 145.6182 70.358) (end 157.226 70.358) (width 0.254) (layer B.Cu) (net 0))
 (segment (start 158.242 68.1355) (end 156.9085 69.596) (width 0.254) (layer B.Cu) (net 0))
 (segment (start 155.956 65.8495) (end 155.7655 65.7225) (width 0.254) (layer B.Cu) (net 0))
 (segment (start 154.686 67.056) (end 155.829 67.056) (width 0.254) (layer B.Cu) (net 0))
 (segment (start 156.9085 69.596) (end 154.6225 69.596) (width 0.254) (layer B.Cu) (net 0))
 (segment (start 154.686 67.818) (end 154.686 67.056) (width 0.254) (layer B.Cu) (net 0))
 (segment (start 156.4005 64.262) (end 153.797 64.262) (width 0.254) (layer B.Cu) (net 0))
 (segment (start 156.591 65.659) (end 156.591 67.3735) (width 0.254) (layer B.Cu) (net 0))
 (segment (start 154.6225 69.596) (end 154.6225 68.707) (width 0.254) (layer B.Cu) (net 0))
 (segment (start 158.1785 64.9605) (end 158.242 68.1355) (width 0.254) (layer B.Cu) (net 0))
 (segment (start 154.6225 68.707) (end 156.5275 68.707) (width 0.254) (layer B.Cu) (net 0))
 (segment (start 157.4165 65.405) (end 156.4005 64.262) (width 0.254) (layer B.Cu) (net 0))
 (segment (start 157.4165 67.8815) (end 157.4165 65.405) (width 0.254) (layer B.Cu) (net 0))
 (segment (start 153.797 65.0875) (end 156.0195 65.0875) (width 0.254) (layer B.Cu) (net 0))
 (segment (start 130.302 64.0715) (end 130.302 68.326) (width 0.254) (layer B.Cu) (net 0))
 (segment (start 135.382 64.0715) (end 135.382 62.9285) (width 0.254) (layer B.Cu) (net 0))
 (segment (start 131.445 62.9285) (end 130.302 64.0715) (width 0.254) (layer B.Cu) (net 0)))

